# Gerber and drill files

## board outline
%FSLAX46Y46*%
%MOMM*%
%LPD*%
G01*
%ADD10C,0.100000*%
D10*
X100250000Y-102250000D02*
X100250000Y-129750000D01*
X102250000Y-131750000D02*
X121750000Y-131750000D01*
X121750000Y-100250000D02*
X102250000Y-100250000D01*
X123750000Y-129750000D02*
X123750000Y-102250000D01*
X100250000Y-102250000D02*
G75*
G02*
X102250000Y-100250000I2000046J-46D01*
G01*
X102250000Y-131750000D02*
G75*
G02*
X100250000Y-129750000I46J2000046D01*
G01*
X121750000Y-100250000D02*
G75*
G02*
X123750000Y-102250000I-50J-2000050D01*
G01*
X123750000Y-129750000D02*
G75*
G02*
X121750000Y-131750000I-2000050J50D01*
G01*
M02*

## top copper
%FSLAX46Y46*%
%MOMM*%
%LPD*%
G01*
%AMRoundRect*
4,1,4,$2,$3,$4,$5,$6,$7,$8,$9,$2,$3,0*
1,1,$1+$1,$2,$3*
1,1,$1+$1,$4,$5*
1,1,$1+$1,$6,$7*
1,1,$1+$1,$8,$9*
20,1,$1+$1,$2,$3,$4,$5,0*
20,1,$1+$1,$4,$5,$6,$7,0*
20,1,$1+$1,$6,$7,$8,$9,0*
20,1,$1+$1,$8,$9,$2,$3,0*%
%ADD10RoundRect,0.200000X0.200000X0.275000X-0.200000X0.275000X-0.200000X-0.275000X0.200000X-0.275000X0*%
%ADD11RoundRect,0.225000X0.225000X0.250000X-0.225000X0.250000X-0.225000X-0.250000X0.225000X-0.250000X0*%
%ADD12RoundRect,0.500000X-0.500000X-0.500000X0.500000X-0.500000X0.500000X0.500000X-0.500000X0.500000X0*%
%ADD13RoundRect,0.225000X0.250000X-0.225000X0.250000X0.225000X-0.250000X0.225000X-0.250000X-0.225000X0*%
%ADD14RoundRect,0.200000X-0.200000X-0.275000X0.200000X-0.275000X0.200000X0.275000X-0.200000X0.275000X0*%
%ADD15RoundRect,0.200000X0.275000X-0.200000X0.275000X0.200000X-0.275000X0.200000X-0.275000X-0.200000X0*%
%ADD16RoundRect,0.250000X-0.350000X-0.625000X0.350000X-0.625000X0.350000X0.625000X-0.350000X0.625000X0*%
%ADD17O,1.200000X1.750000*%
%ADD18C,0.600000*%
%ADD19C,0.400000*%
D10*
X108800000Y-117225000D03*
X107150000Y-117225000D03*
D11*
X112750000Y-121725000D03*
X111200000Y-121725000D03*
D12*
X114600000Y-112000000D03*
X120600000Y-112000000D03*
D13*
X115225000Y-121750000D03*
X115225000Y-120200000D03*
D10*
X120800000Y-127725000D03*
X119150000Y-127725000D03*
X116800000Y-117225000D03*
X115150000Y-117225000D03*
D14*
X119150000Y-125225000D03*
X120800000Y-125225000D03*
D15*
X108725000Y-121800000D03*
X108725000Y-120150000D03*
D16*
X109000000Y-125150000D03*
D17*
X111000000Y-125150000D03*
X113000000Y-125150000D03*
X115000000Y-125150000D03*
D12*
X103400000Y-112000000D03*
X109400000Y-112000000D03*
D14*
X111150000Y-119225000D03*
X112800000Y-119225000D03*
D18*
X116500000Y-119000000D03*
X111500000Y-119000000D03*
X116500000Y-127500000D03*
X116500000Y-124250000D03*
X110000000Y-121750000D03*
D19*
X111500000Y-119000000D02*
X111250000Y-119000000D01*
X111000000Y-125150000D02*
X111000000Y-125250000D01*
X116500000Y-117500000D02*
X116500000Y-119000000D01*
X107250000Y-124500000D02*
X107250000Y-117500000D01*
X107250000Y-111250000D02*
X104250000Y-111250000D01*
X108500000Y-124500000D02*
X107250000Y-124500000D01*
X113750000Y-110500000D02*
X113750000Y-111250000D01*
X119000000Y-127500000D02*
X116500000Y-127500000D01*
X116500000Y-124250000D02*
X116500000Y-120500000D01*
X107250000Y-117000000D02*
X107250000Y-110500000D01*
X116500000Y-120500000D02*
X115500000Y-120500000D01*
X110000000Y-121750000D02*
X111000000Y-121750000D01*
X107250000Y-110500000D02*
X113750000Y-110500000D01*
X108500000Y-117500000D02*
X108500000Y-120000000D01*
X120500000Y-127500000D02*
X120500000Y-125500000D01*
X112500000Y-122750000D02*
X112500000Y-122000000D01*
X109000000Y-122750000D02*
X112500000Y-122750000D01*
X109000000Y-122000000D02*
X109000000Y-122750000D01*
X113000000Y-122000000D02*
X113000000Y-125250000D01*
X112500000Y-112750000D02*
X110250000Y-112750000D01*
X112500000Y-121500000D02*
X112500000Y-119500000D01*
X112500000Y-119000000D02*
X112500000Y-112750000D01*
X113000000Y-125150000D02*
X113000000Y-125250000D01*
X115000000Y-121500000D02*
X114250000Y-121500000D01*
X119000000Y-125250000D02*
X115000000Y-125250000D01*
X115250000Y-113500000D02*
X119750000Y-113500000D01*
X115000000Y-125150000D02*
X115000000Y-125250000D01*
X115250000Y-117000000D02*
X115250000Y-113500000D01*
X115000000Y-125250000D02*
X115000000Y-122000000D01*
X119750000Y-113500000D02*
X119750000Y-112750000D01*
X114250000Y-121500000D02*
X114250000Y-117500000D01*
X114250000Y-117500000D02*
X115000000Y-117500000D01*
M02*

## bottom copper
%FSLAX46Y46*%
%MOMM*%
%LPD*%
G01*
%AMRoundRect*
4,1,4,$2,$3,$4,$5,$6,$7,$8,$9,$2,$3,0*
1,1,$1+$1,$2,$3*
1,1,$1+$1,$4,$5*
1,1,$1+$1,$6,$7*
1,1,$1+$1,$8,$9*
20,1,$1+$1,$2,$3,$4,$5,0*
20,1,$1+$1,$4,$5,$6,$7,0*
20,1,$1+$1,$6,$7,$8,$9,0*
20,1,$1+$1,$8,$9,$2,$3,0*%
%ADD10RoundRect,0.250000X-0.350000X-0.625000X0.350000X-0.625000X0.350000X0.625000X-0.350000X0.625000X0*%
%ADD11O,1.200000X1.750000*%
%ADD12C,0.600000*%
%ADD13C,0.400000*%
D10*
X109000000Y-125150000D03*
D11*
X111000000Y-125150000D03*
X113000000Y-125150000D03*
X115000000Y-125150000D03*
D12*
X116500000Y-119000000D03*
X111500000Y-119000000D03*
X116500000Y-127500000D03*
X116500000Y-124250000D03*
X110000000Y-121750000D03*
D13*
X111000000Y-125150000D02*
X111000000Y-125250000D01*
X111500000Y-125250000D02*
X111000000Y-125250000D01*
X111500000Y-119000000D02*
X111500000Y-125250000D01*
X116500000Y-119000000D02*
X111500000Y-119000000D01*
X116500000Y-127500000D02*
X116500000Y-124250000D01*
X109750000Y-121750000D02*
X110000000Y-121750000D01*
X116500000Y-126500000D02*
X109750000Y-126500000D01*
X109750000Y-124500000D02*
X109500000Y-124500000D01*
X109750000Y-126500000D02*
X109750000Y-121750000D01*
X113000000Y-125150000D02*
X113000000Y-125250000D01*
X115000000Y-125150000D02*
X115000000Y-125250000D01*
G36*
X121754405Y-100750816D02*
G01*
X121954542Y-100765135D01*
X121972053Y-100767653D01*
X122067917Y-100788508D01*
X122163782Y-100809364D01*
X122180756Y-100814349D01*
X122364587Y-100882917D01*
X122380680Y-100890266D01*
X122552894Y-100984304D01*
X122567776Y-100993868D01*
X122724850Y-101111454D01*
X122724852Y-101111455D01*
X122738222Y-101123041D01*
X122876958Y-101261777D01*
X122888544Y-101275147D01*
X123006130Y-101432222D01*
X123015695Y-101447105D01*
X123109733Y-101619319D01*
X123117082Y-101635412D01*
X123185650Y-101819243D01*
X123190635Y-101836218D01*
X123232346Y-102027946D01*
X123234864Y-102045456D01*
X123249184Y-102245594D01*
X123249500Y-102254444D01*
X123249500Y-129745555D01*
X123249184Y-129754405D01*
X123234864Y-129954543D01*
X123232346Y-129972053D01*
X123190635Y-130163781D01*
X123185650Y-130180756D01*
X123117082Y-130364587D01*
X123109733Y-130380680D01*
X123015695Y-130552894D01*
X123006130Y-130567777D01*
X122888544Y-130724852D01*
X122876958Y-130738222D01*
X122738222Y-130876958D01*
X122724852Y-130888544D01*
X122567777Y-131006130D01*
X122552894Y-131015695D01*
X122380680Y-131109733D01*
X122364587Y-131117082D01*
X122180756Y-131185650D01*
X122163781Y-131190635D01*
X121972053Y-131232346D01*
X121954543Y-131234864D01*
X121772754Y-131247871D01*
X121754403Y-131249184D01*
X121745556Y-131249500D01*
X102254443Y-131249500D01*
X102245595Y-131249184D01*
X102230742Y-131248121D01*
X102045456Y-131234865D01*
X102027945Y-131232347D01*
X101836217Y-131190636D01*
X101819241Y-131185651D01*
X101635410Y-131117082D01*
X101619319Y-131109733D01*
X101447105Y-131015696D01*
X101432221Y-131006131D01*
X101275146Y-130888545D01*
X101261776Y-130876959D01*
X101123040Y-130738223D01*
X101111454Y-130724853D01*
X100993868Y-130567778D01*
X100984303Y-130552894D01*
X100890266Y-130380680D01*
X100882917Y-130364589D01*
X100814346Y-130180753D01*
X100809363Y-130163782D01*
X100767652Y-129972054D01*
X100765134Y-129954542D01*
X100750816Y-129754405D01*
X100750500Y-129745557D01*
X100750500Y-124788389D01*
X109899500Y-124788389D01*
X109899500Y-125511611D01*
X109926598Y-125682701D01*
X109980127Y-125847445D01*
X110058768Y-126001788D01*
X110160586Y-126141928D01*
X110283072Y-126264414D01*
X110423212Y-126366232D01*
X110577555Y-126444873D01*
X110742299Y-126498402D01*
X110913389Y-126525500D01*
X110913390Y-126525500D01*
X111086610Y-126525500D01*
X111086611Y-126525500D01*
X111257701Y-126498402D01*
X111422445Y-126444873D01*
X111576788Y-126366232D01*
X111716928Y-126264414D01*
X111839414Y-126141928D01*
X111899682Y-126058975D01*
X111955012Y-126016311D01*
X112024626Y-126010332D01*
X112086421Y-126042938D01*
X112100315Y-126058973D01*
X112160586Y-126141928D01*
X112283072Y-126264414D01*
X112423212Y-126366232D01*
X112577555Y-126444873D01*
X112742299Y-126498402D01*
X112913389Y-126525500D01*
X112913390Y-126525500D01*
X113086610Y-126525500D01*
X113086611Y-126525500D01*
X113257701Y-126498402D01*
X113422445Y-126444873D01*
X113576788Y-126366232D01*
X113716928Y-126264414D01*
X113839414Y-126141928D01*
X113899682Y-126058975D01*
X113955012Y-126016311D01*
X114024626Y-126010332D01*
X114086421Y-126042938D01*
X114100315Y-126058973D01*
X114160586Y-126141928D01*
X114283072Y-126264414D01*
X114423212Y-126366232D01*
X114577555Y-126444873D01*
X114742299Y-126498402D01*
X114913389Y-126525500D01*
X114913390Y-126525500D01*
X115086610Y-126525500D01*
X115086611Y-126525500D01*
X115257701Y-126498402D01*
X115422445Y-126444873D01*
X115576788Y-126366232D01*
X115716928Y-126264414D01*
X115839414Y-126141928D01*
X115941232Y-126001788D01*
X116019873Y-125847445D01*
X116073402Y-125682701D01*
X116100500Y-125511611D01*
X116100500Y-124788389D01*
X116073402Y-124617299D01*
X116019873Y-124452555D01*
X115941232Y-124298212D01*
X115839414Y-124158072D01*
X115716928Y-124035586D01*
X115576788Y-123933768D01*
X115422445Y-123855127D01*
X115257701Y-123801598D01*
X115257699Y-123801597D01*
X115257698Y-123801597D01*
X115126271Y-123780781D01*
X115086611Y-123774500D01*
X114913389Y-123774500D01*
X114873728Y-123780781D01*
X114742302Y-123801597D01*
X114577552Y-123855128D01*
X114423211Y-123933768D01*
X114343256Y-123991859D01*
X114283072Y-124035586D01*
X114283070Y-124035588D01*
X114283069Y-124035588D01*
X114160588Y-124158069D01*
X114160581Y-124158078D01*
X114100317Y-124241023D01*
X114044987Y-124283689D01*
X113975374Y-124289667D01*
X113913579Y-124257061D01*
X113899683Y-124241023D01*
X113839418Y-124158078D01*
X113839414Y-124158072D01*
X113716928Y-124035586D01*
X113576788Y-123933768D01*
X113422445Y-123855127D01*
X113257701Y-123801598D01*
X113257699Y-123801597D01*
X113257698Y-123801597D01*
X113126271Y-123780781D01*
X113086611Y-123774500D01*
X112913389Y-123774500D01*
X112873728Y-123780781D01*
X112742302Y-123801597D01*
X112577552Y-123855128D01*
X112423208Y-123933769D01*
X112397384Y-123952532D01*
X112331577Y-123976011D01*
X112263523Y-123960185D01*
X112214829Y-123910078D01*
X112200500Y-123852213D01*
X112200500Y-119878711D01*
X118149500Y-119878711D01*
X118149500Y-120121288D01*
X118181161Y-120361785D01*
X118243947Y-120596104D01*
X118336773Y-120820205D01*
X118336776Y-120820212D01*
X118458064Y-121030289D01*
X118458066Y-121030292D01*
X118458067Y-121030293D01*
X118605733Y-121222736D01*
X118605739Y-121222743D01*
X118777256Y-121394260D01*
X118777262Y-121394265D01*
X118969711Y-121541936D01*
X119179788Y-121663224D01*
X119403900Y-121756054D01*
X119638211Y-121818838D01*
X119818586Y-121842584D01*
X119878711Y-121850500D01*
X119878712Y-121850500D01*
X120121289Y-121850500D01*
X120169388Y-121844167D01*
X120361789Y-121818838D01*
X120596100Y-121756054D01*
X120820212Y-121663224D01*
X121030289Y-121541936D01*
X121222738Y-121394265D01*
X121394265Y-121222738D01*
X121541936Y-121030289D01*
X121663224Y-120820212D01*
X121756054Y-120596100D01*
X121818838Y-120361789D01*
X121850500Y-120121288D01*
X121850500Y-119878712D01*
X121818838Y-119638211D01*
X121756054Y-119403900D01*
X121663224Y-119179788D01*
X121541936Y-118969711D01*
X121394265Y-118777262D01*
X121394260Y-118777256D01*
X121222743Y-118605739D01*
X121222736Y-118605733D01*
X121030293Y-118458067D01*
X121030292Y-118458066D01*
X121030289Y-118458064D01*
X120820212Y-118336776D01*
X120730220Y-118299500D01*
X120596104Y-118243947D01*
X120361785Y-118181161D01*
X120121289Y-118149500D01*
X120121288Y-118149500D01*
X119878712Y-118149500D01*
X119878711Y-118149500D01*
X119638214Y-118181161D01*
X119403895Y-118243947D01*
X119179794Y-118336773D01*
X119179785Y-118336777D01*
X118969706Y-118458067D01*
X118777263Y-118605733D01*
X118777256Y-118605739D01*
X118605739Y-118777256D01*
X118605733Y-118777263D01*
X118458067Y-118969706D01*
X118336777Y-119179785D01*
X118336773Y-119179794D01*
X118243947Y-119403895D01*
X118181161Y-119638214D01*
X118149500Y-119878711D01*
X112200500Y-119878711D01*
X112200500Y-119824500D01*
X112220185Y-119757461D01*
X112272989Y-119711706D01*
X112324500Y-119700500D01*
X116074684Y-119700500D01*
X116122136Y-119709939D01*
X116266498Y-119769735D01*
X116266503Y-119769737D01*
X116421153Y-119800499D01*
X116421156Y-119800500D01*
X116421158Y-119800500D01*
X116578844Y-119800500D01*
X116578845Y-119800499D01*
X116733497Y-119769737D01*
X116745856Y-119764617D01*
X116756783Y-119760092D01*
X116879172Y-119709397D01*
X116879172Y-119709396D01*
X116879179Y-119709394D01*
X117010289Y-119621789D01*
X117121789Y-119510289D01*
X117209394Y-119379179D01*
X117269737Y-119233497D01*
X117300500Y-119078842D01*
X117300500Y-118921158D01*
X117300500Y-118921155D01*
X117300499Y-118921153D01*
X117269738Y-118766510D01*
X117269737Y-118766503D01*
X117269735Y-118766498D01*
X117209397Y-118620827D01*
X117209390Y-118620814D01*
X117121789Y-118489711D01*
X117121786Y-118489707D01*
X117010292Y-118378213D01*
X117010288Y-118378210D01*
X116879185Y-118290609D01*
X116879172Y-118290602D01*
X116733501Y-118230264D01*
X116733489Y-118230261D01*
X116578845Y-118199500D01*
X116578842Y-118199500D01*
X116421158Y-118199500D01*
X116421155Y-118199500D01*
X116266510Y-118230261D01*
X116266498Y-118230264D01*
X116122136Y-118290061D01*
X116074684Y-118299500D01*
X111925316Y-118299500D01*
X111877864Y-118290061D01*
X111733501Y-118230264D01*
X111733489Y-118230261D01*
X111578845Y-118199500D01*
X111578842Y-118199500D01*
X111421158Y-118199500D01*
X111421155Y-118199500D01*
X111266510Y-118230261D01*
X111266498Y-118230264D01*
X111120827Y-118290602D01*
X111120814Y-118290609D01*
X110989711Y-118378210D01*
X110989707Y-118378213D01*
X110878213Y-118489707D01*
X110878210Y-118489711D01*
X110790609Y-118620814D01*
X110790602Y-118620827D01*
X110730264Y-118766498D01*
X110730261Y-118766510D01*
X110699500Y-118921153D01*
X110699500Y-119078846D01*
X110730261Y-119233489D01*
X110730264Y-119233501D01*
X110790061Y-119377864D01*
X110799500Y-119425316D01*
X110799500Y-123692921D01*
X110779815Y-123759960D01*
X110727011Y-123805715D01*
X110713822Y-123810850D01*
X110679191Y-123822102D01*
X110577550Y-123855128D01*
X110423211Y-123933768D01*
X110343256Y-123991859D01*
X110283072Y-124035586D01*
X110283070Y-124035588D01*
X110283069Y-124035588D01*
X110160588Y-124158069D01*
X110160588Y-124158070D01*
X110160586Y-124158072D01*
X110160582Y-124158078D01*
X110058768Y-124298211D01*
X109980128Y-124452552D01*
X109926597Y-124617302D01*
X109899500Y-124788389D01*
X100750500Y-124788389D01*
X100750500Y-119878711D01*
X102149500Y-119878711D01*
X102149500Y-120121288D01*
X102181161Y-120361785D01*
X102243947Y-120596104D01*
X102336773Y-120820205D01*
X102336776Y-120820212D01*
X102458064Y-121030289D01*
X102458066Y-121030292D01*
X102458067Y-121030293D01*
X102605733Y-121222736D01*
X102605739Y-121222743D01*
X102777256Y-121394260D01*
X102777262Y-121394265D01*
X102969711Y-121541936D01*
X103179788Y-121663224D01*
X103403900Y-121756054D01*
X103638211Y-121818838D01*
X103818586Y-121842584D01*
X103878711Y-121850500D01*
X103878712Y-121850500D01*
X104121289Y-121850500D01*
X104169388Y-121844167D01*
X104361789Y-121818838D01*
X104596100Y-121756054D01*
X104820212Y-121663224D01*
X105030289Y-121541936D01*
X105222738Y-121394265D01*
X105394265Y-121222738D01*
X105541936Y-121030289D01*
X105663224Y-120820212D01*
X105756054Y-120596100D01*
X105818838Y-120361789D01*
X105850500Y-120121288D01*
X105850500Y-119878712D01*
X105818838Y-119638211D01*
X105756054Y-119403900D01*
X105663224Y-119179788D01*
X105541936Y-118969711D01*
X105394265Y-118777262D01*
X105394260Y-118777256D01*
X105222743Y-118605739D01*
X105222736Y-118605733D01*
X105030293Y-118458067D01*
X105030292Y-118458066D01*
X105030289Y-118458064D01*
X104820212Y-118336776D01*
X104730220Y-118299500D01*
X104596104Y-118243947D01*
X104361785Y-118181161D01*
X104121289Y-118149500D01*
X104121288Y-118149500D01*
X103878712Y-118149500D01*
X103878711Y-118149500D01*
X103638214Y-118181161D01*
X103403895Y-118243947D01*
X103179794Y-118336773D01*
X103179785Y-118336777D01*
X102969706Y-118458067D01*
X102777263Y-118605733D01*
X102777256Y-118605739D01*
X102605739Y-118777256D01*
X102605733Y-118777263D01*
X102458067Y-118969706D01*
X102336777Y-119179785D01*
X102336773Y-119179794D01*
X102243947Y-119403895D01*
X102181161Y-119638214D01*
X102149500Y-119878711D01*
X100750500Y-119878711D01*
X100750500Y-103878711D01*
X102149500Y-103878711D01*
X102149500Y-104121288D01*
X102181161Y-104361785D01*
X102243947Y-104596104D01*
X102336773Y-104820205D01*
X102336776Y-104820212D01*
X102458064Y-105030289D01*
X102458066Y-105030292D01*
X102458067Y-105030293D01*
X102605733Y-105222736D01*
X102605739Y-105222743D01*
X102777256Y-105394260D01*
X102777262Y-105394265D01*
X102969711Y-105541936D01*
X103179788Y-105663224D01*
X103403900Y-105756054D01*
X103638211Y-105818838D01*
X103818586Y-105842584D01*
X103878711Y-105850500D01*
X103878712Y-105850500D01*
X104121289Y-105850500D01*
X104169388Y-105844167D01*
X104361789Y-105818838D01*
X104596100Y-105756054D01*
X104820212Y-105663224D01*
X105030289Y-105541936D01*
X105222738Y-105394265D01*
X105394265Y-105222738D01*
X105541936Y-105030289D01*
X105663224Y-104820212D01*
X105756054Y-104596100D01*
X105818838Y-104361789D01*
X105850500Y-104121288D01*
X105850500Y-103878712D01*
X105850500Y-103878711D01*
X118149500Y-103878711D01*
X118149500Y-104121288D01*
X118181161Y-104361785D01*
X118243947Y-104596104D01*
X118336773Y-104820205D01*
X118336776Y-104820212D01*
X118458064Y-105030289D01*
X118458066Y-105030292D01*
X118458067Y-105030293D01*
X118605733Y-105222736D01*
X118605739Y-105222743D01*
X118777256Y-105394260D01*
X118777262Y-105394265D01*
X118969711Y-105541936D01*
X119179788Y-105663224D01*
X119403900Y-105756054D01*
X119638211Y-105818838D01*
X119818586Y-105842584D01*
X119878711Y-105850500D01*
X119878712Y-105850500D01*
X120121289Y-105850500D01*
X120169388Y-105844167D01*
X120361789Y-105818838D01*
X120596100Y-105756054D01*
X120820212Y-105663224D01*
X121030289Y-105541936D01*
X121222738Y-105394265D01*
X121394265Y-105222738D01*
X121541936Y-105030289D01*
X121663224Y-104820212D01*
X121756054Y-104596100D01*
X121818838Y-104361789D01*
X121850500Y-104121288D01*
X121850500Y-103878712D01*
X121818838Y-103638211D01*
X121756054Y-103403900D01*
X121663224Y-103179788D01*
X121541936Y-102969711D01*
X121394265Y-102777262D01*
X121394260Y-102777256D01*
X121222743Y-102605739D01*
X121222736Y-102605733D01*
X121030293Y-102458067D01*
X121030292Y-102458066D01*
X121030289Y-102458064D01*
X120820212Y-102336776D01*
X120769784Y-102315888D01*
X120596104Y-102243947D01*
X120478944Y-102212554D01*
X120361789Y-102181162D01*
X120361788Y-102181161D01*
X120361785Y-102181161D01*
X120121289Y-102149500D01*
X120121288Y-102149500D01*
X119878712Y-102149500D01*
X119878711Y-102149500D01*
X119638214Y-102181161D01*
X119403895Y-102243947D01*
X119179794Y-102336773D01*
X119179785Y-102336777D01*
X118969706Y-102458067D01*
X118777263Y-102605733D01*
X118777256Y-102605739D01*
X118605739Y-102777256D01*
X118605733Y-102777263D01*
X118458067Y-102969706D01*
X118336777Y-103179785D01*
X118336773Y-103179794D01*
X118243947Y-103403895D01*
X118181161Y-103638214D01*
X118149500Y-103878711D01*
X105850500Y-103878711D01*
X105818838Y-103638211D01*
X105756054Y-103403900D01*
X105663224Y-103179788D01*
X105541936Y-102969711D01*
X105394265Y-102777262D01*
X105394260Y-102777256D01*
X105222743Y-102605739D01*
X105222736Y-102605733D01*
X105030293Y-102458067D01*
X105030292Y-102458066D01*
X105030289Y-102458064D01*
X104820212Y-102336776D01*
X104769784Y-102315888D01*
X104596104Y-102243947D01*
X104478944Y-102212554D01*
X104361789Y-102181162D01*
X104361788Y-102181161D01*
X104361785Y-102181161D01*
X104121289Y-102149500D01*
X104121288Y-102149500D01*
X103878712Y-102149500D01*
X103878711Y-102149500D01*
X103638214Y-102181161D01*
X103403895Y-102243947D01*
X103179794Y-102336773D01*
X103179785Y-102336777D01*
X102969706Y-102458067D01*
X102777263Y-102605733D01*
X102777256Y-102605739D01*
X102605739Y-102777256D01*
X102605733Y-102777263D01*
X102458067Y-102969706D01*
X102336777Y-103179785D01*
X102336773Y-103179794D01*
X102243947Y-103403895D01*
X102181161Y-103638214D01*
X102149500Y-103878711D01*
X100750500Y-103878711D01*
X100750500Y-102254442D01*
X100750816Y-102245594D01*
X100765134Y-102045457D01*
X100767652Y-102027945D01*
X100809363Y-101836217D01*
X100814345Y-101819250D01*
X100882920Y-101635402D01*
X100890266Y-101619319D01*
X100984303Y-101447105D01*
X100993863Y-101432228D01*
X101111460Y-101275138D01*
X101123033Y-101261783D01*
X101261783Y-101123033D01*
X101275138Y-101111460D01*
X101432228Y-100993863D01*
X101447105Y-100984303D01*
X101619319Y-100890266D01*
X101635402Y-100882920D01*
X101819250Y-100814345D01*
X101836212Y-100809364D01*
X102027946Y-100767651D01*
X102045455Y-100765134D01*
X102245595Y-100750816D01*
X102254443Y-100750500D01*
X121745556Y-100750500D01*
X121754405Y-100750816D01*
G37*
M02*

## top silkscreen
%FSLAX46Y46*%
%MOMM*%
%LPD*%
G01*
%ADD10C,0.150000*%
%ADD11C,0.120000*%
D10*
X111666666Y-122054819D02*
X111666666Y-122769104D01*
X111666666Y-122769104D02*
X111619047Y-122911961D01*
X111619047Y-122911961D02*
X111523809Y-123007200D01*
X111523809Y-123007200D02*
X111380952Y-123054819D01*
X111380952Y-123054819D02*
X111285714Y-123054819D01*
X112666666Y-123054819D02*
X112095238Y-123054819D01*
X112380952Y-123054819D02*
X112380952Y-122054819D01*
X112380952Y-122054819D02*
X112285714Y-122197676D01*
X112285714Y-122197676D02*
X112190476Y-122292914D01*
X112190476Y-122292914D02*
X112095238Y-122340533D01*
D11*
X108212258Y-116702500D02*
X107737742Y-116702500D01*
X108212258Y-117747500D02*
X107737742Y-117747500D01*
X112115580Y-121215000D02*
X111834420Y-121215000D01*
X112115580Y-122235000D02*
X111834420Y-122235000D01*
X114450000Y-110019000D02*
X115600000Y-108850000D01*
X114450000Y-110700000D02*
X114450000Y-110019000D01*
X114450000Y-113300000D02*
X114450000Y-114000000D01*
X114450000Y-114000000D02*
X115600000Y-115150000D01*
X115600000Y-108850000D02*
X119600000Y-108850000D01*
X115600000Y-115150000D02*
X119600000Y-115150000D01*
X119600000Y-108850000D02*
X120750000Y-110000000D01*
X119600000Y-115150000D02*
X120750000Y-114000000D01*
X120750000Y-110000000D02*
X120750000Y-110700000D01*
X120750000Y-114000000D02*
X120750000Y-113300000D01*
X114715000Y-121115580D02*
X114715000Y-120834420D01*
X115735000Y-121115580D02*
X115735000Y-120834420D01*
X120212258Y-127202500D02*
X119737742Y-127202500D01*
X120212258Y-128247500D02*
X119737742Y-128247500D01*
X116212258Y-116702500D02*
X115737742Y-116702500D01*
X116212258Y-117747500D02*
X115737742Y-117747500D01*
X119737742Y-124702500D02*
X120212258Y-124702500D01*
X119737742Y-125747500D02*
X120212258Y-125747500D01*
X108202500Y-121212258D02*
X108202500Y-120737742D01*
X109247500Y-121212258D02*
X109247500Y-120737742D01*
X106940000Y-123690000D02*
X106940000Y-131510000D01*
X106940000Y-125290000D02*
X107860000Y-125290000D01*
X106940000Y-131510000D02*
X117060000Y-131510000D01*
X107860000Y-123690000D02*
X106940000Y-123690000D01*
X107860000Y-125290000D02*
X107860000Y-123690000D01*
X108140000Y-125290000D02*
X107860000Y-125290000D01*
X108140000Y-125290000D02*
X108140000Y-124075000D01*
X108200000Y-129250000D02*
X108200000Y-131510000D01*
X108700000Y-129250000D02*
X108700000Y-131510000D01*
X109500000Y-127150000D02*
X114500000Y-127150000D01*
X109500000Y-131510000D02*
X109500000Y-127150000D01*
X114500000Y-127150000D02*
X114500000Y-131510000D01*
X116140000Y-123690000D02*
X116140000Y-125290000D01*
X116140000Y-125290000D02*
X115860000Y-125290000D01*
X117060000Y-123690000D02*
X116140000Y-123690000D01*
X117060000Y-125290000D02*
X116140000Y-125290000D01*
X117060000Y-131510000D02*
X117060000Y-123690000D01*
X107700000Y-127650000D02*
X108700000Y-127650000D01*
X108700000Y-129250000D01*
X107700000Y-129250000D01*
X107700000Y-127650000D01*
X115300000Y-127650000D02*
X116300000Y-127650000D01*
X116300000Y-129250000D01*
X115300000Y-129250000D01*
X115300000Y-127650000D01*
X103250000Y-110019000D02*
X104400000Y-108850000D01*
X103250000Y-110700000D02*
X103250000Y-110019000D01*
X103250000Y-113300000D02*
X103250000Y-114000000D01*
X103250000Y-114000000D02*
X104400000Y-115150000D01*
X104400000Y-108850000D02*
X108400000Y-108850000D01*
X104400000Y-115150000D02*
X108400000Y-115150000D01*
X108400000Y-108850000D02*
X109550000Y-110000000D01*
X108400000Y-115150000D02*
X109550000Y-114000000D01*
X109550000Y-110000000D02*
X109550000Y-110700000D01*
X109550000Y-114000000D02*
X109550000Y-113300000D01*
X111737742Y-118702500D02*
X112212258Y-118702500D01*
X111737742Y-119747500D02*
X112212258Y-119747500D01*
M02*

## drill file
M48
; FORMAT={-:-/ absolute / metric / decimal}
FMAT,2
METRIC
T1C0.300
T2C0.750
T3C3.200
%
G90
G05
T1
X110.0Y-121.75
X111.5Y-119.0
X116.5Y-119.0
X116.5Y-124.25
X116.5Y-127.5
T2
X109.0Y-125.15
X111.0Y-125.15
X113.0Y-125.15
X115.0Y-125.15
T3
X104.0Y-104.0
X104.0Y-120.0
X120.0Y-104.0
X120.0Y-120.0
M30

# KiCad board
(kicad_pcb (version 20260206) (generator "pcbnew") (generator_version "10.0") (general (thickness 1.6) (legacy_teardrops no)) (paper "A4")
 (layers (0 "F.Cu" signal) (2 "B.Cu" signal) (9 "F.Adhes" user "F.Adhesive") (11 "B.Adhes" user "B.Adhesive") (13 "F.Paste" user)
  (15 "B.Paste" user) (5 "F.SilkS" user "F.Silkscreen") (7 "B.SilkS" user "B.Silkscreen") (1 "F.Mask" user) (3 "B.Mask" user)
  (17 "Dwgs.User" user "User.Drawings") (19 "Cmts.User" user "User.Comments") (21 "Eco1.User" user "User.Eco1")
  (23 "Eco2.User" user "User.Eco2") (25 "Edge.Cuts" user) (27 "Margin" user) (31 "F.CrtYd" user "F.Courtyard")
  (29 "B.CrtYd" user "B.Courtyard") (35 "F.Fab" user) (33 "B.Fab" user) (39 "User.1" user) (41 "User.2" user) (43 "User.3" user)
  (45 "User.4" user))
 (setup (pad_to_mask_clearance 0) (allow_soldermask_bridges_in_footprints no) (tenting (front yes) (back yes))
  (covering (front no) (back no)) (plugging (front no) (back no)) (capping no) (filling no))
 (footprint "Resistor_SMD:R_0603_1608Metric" (layer "F.Cu") (at 107.975 117.225 180)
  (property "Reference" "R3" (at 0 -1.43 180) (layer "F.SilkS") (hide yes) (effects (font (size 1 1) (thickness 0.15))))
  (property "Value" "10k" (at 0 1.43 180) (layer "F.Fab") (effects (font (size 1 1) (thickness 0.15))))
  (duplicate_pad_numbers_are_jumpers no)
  (fp_line (start -0.237258 0.5225) (end 0.237258 0.5225) (stroke (width 0.12) (type solid)) (layer "F.SilkS"))
  (fp_line (start -0.237258 -0.5225) (end 0.237258 -0.5225) (stroke (width 0.12) (type solid)) (layer "F.SilkS"))
  (pad "1" smd roundrect (at -0.825 0 180) (size 0.8 0.95) (layers "F.Cu" "F.Mask" "F.Paste") (roundrect_rratio 0.25) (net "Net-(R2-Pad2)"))
  (pad "2" smd roundrect (at 0.825 0 180) (size 0.8 0.95) (layers "F.Cu" "F.Mask" "F.Paste") (roundrect_rratio 0.25) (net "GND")))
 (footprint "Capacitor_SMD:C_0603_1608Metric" (layer "F.Cu") (at 111.975 121.725 180)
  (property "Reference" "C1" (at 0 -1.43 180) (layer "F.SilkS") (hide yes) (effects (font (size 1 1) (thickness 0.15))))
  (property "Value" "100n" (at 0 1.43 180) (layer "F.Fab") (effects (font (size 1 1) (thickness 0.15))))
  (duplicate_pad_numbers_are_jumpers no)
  (fp_line (start -0.14058 0.51) (end 0.14058 0.51) (stroke (width 0.12) (type solid)) (layer "F.SilkS"))
  (fp_line (start -0.14058 -0.51) (end 0.14058 -0.51) (stroke (width 0.12) (type solid)) (layer "F.SilkS"))
  (pad "1" smd roundrect (at -0.775 0 180) (size 0.9 0.95) (layers "F.Cu" "F.Mask" "F.Paste") (roundrect_rratio 0.25) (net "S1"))
  (pad "2" smd roundrect (at 0.775 0 180) (size 0.9 0.95) (layers "F.Cu" "F.Mask" "F.Paste") (roundrect_rratio 0.25) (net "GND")))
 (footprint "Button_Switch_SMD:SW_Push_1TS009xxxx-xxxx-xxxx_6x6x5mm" (layer "F.Cu") (at 117.6 112)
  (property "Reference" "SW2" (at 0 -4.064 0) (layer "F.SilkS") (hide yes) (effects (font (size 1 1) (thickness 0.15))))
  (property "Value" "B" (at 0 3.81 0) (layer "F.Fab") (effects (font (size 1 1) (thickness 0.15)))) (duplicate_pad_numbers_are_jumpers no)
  (fp_line (start -3.15 -1.981) (end -2 -3.15) (stroke (width 0.12) (type default)) (layer "F.SilkS"))
  (fp_line (start -3.15 -1.3) (end -3.15 -1.981) (stroke (width 0.12) (type default)) (layer "F.SilkS"))
  (fp_line (start -3.15 1.3) (end -3.15 2) (stroke (width 0.12) (type default)) (layer "F.SilkS"))
  (fp_line (start -3.15 2) (end -2 3.15) (stroke (width 0.12) (type default)) (layer "F.SilkS"))
  (fp_line (start -2 -3.15) (end 2 -3.15) (stroke (width 0.12) (type default)) (layer "F.SilkS"))
  (fp_line (start -2 3.15) (end 2 3.15) (stroke (width 0.12) (type default)) (layer "F.SilkS"))
  (fp_line (start 2 -3.15) (end 3.15 -2) (stroke (width 0.12) (type default)) (layer "F.SilkS"))
  (fp_line (start 2 3.15) (end 3.15 2) (stroke (width 0.12) (type default)) (layer "F.SilkS"))
  (fp_line (start 3.15 -2) (end 3.15 -1.3) (stroke (width 0.12) (type default)) (layer "F.SilkS"))
  (fp_line (start 3.15 2) (end 3.15 1.3) (stroke (width 0.12) (type default)) (layer "F.SilkS"))
  (pad "1" smd roundrect (at -3 0) (size 2 2) (layers "F.Cu" "F.Mask" "F.Paste") (roundrect_rratio 0.25) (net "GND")
   (thermal_bridge_angle 45))
  (pad "2" smd roundrect (at 3 0) (size 2 2) (layers "F.Cu" "F.Mask" "F.Paste") (roundrect_rratio 0.25) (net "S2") (thermal_bridge_angle 45)))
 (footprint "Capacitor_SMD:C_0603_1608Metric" (layer "F.Cu") (at 115.225 120.975 90)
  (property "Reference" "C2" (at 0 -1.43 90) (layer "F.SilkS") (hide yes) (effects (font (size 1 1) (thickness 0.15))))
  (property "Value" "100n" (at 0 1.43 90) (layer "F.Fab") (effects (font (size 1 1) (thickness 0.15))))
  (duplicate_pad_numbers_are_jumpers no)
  (fp_line (start -0.14058 -0.51) (end 0.14058 -0.51) (stroke (width 0.12) (type solid)) (layer "F.SilkS"))
  (fp_line (start -0.14058 0.51) (end 0.14058 0.51) (stroke (width 0.12) (type solid)) (layer "F.SilkS"))
  (pad "1" smd roundrect (at -0.775 0 90) (size 0.9 0.95) (layers "F.Cu" "F.Mask" "F.Paste") (roundrect_rratio 0.25) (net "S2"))
  (pad "2" smd roundrect (at 0.775 0 90) (size 0.9 0.95) (layers "F.Cu" "F.Mask" "F.Paste") (roundrect_rratio 0.25) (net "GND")))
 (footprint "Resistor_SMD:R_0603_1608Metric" (layer "F.Cu") (at 119.975 127.725 180)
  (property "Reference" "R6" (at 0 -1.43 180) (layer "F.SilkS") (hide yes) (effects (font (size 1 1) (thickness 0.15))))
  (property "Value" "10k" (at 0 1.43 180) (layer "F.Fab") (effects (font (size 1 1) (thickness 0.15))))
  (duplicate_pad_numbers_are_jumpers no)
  (fp_line (start -0.237258 0.5225) (end 0.237258 0.5225) (stroke (width 0.12) (type solid)) (layer "F.SilkS"))
  (fp_line (start -0.237258 -0.5225) (end 0.237258 -0.5225) (stroke (width 0.12) (type solid)) (layer "F.SilkS"))
  (pad "1" smd roundrect (at -0.825 0 180) (size 0.8 0.95) (layers "F.Cu" "F.Mask" "F.Paste") (roundrect_rratio 0.25) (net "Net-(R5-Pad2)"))
  (pad "2" smd roundrect (at 0.825 0 180) (size 0.8 0.95) (layers "F.Cu" "F.Mask" "F.Paste") (roundrect_rratio 0.25) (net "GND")))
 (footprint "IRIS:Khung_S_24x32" (layer "F.Cu") (at 100 132)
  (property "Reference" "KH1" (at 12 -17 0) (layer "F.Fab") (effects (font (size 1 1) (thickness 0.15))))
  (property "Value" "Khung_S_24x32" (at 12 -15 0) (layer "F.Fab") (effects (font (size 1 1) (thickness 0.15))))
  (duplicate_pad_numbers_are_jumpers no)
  (fp_line (start 0.25 -29.75) (end 0.25 -2.25) (stroke (width 0.1) (type solid)) (layer "Edge.Cuts"))
  (fp_line (start 2.25 -0.25) (end 21.75 -0.25) (stroke (width 0.1) (type solid)) (layer "Edge.Cuts"))
  (fp_line (start 21.75 -31.75) (end 2.25 -31.75) (stroke (width 0.1) (type solid)) (layer "Edge.Cuts"))
  (fp_line (start 23.75 -2.25) (end 23.75 -29.75) (stroke (width 0.1) (type solid)) (layer "Edge.Cuts"))
  (fp_arc (start 0.25 -29.75) (mid 0.8358 -31.1642) (end 2.25 -31.75) (stroke (width 0.1) (type solid)) (layer "Edge.Cuts"))
  (fp_arc (start 2.25 -0.25) (mid 0.8358 -0.8358) (end 0.25 -2.25) (stroke (width 0.1) (type solid)) (layer "Edge.Cuts"))
  (fp_arc (start 21.75 -31.75) (mid 23.164199 -31.164199) (end 23.75 -29.75) (stroke (width 0.1) (type solid)) (layer "Edge.Cuts"))
  (fp_arc (start 23.75 -2.25) (mid 23.164199 -0.835801) (end 21.75 -0.25) (stroke (width 0.1) (type solid)) (layer "Edge.Cuts"))
  (pad "" np_thru_hole circle (at 4 -28) (size 3.2 3.2) (drill 3.2) (layers "*.Cu" "*.Mask"))
  (pad "" np_thru_hole circle (at 4 -12) (size 3.2 3.2) (drill 3.2) (layers "*.Cu" "*.Mask"))
  (pad "" np_thru_hole circle (at 20 -28) (size 3.2 3.2) (drill 3.2) (layers "*.Cu" "*.Mask"))
  (pad "" np_thru_hole circle (at 20 -12) (size 3.2 3.2) (drill 3.2) (layers "*.Cu" "*.Mask")))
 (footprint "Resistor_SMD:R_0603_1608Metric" (layer "F.Cu") (at 115.975 117.225 180)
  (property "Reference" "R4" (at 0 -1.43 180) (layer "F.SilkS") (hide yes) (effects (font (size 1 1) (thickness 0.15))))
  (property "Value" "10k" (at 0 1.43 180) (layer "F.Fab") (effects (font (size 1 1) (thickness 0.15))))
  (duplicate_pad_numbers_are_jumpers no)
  (fp_line (start -0.237258 0.5225) (end 0.237258 0.5225) (stroke (width 0.12) (type solid)) (layer "F.SilkS"))
  (fp_line (start -0.237258 -0.5225) (end 0.237258 -0.5225) (stroke (width 0.12) (type solid)) (layer "F.SilkS"))
  (pad "1" smd roundrect (at -0.825 0 180) (size 0.8 0.95) (layers "F.Cu" "F.Mask" "F.Paste") (roundrect_rratio 0.25) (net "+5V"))
  (pad "2" smd roundrect (at 0.825 0 180) (size 0.8 0.95) (layers "F.Cu" "F.Mask" "F.Paste") (roundrect_rratio 0.25) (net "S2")))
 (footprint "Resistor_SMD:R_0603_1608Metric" (layer "F.Cu") (at 119.975 125.225)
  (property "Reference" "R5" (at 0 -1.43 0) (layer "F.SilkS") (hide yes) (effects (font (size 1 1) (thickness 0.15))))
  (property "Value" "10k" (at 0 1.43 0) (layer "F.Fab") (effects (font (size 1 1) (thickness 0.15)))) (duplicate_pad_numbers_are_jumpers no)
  (fp_line (start -0.237258 -0.5225) (end 0.237258 -0.5225) (stroke (width 0.12) (type solid)) (layer "F.SilkS"))
  (fp_line (start -0.237258 0.5225) (end 0.237258 0.5225) (stroke (width 0.12) (type solid)) (layer "F.SilkS"))
  (pad "1" smd roundrect (at -0.825 0) (size 0.8 0.95) (layers "F.Cu" "F.Mask" "F.Paste") (roundrect_rratio 0.25) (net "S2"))
  (pad "2" smd roundrect (at 0.825 0) (size 0.8 0.95) (layers "F.Cu" "F.Mask" "F.Paste") (roundrect_rratio 0.25) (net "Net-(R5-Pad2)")))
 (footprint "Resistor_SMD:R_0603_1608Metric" (layer "F.Cu") (at 108.725 120.975 90)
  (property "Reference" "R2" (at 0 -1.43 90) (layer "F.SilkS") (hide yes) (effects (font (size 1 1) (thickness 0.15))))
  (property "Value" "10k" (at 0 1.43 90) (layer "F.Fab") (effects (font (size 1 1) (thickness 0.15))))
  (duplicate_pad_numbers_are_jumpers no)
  (fp_line (start -0.237258 -0.5225) (end 0.237258 -0.5225) (stroke (width 0.12) (type solid)) (layer "F.SilkS"))
  (fp_line (start -0.237258 0.5225) (end 0.237258 0.5225) (stroke (width 0.12) (type solid)) (layer "F.SilkS"))
  (pad "1" smd roundrect (at -0.825 0 90) (size 0.8 0.95) (layers "F.Cu" "F.Mask" "F.Paste") (roundrect_rratio 0.25) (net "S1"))
  (pad "2" smd roundrect (at 0.825 0 90) (size 0.8 0.95) (layers "F.Cu" "F.Mask" "F.Paste") (roundrect_rratio 0.25) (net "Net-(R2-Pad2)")))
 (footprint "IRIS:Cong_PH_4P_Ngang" (layer "F.Cu") (at 109 125.15)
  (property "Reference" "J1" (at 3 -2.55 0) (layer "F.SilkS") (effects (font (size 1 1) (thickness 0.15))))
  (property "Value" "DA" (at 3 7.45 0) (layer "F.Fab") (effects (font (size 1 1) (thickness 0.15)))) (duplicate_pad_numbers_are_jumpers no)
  (fp_line (start -2.06 -1.46) (end -2.06 6.36) (stroke (width 0.12) (type solid)) (layer "F.SilkS"))
  (fp_line (start -2.06 0.14) (end -1.14 0.14) (stroke (width 0.12) (type solid)) (layer "F.SilkS"))
  (fp_line (start -2.06 6.36) (end 8.06 6.36) (stroke (width 0.12) (type solid)) (layer "F.SilkS"))
  (fp_line (start -1.14 -1.46) (end -2.06 -1.46) (stroke (width 0.12) (type solid)) (layer "F.SilkS"))
  (fp_line (start -1.14 0.14) (end -1.14 -1.46) (stroke (width 0.12) (type solid)) (layer "F.SilkS"))
  (fp_line (start -0.86 0.14) (end -1.14 0.14) (stroke (width 0.12) (type solid)) (layer "F.SilkS"))
  (fp_line (start -0.86 0.14) (end -0.86 -1.075) (stroke (width 0.12) (type solid)) (layer "F.SilkS"))
  (fp_line (start -0.8 4.1) (end -0.8 6.36) (stroke (width 0.12) (type solid)) (layer "F.SilkS"))
  (fp_line (start -0.3 4.1) (end -0.3 6.36) (stroke (width 0.12) (type solid)) (layer "F.SilkS"))
  (fp_line (start 0.5 2) (end 5.5 2) (stroke (width 0.12) (type solid)) (layer "F.SilkS"))
  (fp_line (start 0.5 6.36) (end 0.5 2) (stroke (width 0.12) (type solid)) (layer "F.SilkS"))
  (fp_line (start 5.5 2) (end 5.5 6.36) (stroke (width 0.12) (type solid)) (layer "F.SilkS"))
  (fp_line (start 7.14 -1.46) (end 7.14 0.14) (stroke (width 0.12) (type solid)) (layer "F.SilkS"))
  (fp_line (start 7.14 0.14) (end 6.86 0.14) (stroke (width 0.12) (type solid)) (layer "F.SilkS"))
  (fp_line (start 8.06 -1.46) (end 7.14 -1.46) (stroke (width 0.12) (type solid)) (layer "F.SilkS"))
  (fp_line (start 8.06 0.14) (end 7.14 0.14) (stroke (width 0.12) (type solid)) (layer "F.SilkS"))
  (fp_line (start 8.06 6.36) (end 8.06 -1.46) (stroke (width 0.12) (type solid)) (layer "F.SilkS"))
  (fp_rect (start -1.3 2.5) (end -0.3 4.1) (stroke (width 0.12) (type solid)) (fill no) (layer "F.SilkS"))
  (fp_rect (start 6.3 2.5) (end 7.3 4.1) (stroke (width 0.12) (type solid)) (fill no) (layer "F.SilkS"))
  (pad "1" thru_hole roundrect (at 0 0) (size 1.2 1.75) (drill 0.75) (layers "*.Cu" "*.Mask") (remove_unused_layers no)
   (roundrect_rratio 0.208333) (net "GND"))
  (pad "2" thru_hole oval (at 2 0) (size 1.2 1.75) (drill 0.75) (layers "*.Cu" "*.Mask") (remove_unused_layers no) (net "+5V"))
  (pad "3" thru_hole oval (at 4 0) (size 1.2 1.75) (drill 0.75) (layers "*.Cu" "*.Mask") (remove_unused_layers no) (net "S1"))
  (pad "4" thru_hole oval (at 6 0) (size 1.2 1.75) (drill 0.75) (layers "*.Cu" "*.Mask") (remove_unused_layers no) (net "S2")))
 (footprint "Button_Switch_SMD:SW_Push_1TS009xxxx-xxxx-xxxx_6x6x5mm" (layer "F.Cu") (at 106.4 112)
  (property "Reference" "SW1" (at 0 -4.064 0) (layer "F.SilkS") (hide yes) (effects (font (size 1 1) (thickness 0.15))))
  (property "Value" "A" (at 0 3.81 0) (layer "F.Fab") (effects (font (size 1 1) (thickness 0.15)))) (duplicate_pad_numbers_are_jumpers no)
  (fp_line (start -3.15 -1.981) (end -2 -3.15) (stroke (width 0.12) (type default)) (layer "F.SilkS"))
  (fp_line (start -3.15 -1.3) (end -3.15 -1.981) (stroke (width 0.12) (type default)) (layer "F.SilkS"))
  (fp_line (start -3.15 1.3) (end -3.15 2) (stroke (width 0.12) (type default)) (layer "F.SilkS"))
  (fp_line (start -3.15 2) (end -2 3.15) (stroke (width 0.12) (type default)) (layer "F.SilkS"))
  (fp_line (start -2 -3.15) (end 2 -3.15) (stroke (width 0.12) (type default)) (layer "F.SilkS"))
  (fp_line (start -2 3.15) (end 2 3.15) (stroke (width 0.12) (type default)) (layer "F.SilkS"))
  (fp_line (start 2 -3.15) (end 3.15 -2) (stroke (width 0.12) (type default)) (layer "F.SilkS"))
  (fp_line (start 2 3.15) (end 3.15 2) (stroke (width 0.12) (type default)) (layer "F.SilkS"))
  (fp_line (start 3.15 -2) (end 3.15 -1.3) (stroke (width 0.12) (type default)) (layer "F.SilkS"))
  (fp_line (start 3.15 2) (end 3.15 1.3) (stroke (width 0.12) (type default)) (layer "F.SilkS"))
  (pad "1" smd roundrect (at -3 0) (size 2 2) (layers "F.Cu" "F.Mask" "F.Paste") (roundrect_rratio 0.25) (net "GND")
   (thermal_bridge_angle 45))
  (pad "2" smd roundrect (at 3 0) (size 2 2) (layers "F.Cu" "F.Mask" "F.Paste") (roundrect_rratio 0.25) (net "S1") (thermal_bridge_angle 45)))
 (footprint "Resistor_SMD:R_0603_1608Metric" (layer "F.Cu") (at 111.975 119.225)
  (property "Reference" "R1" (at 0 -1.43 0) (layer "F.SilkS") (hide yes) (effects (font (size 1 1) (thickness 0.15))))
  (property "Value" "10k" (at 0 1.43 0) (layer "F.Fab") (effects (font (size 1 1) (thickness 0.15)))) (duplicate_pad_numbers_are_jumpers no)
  (fp_line (start -0.237258 -0.5225) (end 0.237258 -0.5225) (stroke (width 0.12) (type solid)) (layer "F.SilkS"))
  (fp_line (start -0.237258 0.5225) (end 0.237258 0.5225) (stroke (width 0.12) (type solid)) (layer "F.SilkS"))
  (pad "1" smd roundrect (at -0.825 0) (size 0.8 0.95) (layers "F.Cu" "F.Mask" "F.Paste") (roundrect_rratio 0.25) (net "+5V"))
  (pad "2" smd roundrect (at 0.825 0) (size 0.8 0.95) (layers "F.Cu" "F.Mask" "F.Paste") (roundrect_rratio 0.25) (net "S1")))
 (segment (start 111.5 119) (end 111.25 119) (width 0.4) (layer "F.Cu") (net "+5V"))
 (segment (start 111 125.15) (end 111 125.25) (width 0.4) (layer "F.Cu") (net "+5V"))
 (segment (start 116.5 117.5) (end 116.5 119) (width 0.4) (layer "F.Cu") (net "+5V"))
 (via (at 116.5 119) (size 0.6) (drill 0.3) (layers "F.Cu" "B.Cu") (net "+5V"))
 (via (at 111.5 119) (size 0.6) (drill 0.3) (layers "F.Cu" "B.Cu") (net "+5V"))
 (segment (start 111 125.15) (end 111 125.25) (width 0.4) (layer "B.Cu") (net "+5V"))
 (segment (start 111.5 125.25) (end 111 125.25) (width 0.4) (layer "B.Cu") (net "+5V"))
 (segment (start 111.5 119) (end 111.5 125.25) (width 0.4) (layer "B.Cu") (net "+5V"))
 (segment (start 116.5 119) (end 111.5 119) (width 0.4) (layer "B.Cu") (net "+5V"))
 (segment (start 107.25 124.5) (end 107.25 117.5) (width 0.4) (layer "F.Cu") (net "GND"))
 (segment (start 107.25 111.25) (end 104.25 111.25) (width 0.4) (layer "F.Cu") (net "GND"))
 (segment (start 108.5 124.5) (end 107.25 124.5) (width 0.4) (layer "F.Cu") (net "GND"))
 (segment (start 113.75 110.5) (end 113.75 111.25) (width 0.4) (layer "F.Cu") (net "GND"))
 (segment (start 119 127.5) (end 116.5 127.5) (width 0.4) (layer "F.Cu") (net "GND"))
 (segment (start 116.5 124.25) (end 116.5 120.5) (width 0.4) (layer "F.Cu") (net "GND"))
 (segment (start 107.25 117) (end 107.25 110.5) (width 0.4) (layer "F.Cu") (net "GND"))
 (segment (start 116.5 120.5) (end 115.5 120.5) (width 0.4) (layer "F.Cu") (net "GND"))
 (segment (start 110 121.75) (end 111 121.75) (width 0.4) (layer "F.Cu") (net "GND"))
 (segment (start 107.25 110.5) (end 113.75 110.5) (width 0.4) (layer "F.Cu") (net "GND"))
 (via (at 116.5 127.5) (size 0.6) (drill 0.3) (layers "F.Cu" "B.Cu") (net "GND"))
 (via (at 116.5 124.25) (size 0.6) (drill 0.3) (layers "F.Cu" "B.Cu") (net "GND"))
 (via (at 110 121.75) (size 0.6) (drill 0.3) (layers "F.Cu" "B.Cu") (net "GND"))
 (segment (start 116.5 127.5) (end 116.5 124.25) (width 0.4) (layer "B.Cu") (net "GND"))
 (segment (start 109.75 121.75) (end 110 121.75) (width 0.4) (layer "B.Cu") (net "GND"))
 (segment (start 116.5 126.5) (end 109.75 126.5) (width 0.4) (layer "B.Cu") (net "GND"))
 (segment (start 109.75 124.5) (end 109.5 124.5) (width 0.4) (layer "B.Cu") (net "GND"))
 (segment (start 109.75 126.5) (end 109.75 121.75) (width 0.4) (layer "B.Cu") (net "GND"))
 (segment (start 108.5 117.5) (end 108.5 120) (width 0.4) (layer "F.Cu") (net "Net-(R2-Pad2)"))
 (segment (start 120.5 127.5) (end 120.5 125.5) (width 0.4) (layer "F.Cu") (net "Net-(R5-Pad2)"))
 (segment (start 112.5 122.75) (end 112.5 122) (width 0.4) (layer "F.Cu") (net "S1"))
 (segment (start 109 122.75) (end 112.5 122.75) (width 0.4) (layer "F.Cu") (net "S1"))
 (segment (start 109 122) (end 109 122.75) (width 0.4) (layer "F.Cu") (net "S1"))
 (segment (start 113 122) (end 113 125.25) (width 0.4) (layer "F.Cu") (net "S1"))
 (segment (start 112.5 112.75) (end 110.25 112.75) (width 0.4) (layer "F.Cu") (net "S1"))
 (segment (start 112.5 121.5) (end 112.5 119.5) (width 0.4) (layer "F.Cu") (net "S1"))
 (segment (start 112.5 119) (end 112.5 112.75) (width 0.4) (layer "F.Cu") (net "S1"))
 (segment (start 113 125.15) (end 113 125.25) (width 0.4) (layer "F.Cu") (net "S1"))
 (segment (start 113 125.15) (end 113 125.25) (width 0.4) (layer "B.Cu") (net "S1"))
 (segment (start 115 121.5) (end 114.25 121.5) (width 0.4) (layer "F.Cu") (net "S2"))
 (segment (start 119 125.25) (end 115 125.25) (width 0.4) (layer "F.Cu") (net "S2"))
 (segment (start 115.25 113.5) (end 119.75 113.5) (width 0.4) (layer "F.Cu") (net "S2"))
 (segment (start 115 125.15) (end 115 125.25) (width 0.4) (layer "F.Cu") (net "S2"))
 (segment (start 115.25 117) (end 115.25 113.5) (width 0.4) (layer "F.Cu") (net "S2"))
 (segment (start 115 125.25) (end 115 122) (width 0.4) (layer "F.Cu") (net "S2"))
 (segment (start 119.75 113.5) (end 119.75 112.75) (width 0.4) (layer "F.Cu") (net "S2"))
 (segment (start 114.25 121.5) (end 114.25 117.5) (width 0.4) (layer "F.Cu") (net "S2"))
 (segment (start 114.25 117.5) (end 115 117.5) (width 0.4) (layer "F.Cu") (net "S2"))
 (segment (start 115 125.15) (end 115 125.25) (width 0.4) (layer "B.Cu") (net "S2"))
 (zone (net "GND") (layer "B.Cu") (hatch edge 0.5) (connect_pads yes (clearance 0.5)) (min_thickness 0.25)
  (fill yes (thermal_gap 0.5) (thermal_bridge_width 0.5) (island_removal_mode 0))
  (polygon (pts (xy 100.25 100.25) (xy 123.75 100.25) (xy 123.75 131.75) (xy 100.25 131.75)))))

